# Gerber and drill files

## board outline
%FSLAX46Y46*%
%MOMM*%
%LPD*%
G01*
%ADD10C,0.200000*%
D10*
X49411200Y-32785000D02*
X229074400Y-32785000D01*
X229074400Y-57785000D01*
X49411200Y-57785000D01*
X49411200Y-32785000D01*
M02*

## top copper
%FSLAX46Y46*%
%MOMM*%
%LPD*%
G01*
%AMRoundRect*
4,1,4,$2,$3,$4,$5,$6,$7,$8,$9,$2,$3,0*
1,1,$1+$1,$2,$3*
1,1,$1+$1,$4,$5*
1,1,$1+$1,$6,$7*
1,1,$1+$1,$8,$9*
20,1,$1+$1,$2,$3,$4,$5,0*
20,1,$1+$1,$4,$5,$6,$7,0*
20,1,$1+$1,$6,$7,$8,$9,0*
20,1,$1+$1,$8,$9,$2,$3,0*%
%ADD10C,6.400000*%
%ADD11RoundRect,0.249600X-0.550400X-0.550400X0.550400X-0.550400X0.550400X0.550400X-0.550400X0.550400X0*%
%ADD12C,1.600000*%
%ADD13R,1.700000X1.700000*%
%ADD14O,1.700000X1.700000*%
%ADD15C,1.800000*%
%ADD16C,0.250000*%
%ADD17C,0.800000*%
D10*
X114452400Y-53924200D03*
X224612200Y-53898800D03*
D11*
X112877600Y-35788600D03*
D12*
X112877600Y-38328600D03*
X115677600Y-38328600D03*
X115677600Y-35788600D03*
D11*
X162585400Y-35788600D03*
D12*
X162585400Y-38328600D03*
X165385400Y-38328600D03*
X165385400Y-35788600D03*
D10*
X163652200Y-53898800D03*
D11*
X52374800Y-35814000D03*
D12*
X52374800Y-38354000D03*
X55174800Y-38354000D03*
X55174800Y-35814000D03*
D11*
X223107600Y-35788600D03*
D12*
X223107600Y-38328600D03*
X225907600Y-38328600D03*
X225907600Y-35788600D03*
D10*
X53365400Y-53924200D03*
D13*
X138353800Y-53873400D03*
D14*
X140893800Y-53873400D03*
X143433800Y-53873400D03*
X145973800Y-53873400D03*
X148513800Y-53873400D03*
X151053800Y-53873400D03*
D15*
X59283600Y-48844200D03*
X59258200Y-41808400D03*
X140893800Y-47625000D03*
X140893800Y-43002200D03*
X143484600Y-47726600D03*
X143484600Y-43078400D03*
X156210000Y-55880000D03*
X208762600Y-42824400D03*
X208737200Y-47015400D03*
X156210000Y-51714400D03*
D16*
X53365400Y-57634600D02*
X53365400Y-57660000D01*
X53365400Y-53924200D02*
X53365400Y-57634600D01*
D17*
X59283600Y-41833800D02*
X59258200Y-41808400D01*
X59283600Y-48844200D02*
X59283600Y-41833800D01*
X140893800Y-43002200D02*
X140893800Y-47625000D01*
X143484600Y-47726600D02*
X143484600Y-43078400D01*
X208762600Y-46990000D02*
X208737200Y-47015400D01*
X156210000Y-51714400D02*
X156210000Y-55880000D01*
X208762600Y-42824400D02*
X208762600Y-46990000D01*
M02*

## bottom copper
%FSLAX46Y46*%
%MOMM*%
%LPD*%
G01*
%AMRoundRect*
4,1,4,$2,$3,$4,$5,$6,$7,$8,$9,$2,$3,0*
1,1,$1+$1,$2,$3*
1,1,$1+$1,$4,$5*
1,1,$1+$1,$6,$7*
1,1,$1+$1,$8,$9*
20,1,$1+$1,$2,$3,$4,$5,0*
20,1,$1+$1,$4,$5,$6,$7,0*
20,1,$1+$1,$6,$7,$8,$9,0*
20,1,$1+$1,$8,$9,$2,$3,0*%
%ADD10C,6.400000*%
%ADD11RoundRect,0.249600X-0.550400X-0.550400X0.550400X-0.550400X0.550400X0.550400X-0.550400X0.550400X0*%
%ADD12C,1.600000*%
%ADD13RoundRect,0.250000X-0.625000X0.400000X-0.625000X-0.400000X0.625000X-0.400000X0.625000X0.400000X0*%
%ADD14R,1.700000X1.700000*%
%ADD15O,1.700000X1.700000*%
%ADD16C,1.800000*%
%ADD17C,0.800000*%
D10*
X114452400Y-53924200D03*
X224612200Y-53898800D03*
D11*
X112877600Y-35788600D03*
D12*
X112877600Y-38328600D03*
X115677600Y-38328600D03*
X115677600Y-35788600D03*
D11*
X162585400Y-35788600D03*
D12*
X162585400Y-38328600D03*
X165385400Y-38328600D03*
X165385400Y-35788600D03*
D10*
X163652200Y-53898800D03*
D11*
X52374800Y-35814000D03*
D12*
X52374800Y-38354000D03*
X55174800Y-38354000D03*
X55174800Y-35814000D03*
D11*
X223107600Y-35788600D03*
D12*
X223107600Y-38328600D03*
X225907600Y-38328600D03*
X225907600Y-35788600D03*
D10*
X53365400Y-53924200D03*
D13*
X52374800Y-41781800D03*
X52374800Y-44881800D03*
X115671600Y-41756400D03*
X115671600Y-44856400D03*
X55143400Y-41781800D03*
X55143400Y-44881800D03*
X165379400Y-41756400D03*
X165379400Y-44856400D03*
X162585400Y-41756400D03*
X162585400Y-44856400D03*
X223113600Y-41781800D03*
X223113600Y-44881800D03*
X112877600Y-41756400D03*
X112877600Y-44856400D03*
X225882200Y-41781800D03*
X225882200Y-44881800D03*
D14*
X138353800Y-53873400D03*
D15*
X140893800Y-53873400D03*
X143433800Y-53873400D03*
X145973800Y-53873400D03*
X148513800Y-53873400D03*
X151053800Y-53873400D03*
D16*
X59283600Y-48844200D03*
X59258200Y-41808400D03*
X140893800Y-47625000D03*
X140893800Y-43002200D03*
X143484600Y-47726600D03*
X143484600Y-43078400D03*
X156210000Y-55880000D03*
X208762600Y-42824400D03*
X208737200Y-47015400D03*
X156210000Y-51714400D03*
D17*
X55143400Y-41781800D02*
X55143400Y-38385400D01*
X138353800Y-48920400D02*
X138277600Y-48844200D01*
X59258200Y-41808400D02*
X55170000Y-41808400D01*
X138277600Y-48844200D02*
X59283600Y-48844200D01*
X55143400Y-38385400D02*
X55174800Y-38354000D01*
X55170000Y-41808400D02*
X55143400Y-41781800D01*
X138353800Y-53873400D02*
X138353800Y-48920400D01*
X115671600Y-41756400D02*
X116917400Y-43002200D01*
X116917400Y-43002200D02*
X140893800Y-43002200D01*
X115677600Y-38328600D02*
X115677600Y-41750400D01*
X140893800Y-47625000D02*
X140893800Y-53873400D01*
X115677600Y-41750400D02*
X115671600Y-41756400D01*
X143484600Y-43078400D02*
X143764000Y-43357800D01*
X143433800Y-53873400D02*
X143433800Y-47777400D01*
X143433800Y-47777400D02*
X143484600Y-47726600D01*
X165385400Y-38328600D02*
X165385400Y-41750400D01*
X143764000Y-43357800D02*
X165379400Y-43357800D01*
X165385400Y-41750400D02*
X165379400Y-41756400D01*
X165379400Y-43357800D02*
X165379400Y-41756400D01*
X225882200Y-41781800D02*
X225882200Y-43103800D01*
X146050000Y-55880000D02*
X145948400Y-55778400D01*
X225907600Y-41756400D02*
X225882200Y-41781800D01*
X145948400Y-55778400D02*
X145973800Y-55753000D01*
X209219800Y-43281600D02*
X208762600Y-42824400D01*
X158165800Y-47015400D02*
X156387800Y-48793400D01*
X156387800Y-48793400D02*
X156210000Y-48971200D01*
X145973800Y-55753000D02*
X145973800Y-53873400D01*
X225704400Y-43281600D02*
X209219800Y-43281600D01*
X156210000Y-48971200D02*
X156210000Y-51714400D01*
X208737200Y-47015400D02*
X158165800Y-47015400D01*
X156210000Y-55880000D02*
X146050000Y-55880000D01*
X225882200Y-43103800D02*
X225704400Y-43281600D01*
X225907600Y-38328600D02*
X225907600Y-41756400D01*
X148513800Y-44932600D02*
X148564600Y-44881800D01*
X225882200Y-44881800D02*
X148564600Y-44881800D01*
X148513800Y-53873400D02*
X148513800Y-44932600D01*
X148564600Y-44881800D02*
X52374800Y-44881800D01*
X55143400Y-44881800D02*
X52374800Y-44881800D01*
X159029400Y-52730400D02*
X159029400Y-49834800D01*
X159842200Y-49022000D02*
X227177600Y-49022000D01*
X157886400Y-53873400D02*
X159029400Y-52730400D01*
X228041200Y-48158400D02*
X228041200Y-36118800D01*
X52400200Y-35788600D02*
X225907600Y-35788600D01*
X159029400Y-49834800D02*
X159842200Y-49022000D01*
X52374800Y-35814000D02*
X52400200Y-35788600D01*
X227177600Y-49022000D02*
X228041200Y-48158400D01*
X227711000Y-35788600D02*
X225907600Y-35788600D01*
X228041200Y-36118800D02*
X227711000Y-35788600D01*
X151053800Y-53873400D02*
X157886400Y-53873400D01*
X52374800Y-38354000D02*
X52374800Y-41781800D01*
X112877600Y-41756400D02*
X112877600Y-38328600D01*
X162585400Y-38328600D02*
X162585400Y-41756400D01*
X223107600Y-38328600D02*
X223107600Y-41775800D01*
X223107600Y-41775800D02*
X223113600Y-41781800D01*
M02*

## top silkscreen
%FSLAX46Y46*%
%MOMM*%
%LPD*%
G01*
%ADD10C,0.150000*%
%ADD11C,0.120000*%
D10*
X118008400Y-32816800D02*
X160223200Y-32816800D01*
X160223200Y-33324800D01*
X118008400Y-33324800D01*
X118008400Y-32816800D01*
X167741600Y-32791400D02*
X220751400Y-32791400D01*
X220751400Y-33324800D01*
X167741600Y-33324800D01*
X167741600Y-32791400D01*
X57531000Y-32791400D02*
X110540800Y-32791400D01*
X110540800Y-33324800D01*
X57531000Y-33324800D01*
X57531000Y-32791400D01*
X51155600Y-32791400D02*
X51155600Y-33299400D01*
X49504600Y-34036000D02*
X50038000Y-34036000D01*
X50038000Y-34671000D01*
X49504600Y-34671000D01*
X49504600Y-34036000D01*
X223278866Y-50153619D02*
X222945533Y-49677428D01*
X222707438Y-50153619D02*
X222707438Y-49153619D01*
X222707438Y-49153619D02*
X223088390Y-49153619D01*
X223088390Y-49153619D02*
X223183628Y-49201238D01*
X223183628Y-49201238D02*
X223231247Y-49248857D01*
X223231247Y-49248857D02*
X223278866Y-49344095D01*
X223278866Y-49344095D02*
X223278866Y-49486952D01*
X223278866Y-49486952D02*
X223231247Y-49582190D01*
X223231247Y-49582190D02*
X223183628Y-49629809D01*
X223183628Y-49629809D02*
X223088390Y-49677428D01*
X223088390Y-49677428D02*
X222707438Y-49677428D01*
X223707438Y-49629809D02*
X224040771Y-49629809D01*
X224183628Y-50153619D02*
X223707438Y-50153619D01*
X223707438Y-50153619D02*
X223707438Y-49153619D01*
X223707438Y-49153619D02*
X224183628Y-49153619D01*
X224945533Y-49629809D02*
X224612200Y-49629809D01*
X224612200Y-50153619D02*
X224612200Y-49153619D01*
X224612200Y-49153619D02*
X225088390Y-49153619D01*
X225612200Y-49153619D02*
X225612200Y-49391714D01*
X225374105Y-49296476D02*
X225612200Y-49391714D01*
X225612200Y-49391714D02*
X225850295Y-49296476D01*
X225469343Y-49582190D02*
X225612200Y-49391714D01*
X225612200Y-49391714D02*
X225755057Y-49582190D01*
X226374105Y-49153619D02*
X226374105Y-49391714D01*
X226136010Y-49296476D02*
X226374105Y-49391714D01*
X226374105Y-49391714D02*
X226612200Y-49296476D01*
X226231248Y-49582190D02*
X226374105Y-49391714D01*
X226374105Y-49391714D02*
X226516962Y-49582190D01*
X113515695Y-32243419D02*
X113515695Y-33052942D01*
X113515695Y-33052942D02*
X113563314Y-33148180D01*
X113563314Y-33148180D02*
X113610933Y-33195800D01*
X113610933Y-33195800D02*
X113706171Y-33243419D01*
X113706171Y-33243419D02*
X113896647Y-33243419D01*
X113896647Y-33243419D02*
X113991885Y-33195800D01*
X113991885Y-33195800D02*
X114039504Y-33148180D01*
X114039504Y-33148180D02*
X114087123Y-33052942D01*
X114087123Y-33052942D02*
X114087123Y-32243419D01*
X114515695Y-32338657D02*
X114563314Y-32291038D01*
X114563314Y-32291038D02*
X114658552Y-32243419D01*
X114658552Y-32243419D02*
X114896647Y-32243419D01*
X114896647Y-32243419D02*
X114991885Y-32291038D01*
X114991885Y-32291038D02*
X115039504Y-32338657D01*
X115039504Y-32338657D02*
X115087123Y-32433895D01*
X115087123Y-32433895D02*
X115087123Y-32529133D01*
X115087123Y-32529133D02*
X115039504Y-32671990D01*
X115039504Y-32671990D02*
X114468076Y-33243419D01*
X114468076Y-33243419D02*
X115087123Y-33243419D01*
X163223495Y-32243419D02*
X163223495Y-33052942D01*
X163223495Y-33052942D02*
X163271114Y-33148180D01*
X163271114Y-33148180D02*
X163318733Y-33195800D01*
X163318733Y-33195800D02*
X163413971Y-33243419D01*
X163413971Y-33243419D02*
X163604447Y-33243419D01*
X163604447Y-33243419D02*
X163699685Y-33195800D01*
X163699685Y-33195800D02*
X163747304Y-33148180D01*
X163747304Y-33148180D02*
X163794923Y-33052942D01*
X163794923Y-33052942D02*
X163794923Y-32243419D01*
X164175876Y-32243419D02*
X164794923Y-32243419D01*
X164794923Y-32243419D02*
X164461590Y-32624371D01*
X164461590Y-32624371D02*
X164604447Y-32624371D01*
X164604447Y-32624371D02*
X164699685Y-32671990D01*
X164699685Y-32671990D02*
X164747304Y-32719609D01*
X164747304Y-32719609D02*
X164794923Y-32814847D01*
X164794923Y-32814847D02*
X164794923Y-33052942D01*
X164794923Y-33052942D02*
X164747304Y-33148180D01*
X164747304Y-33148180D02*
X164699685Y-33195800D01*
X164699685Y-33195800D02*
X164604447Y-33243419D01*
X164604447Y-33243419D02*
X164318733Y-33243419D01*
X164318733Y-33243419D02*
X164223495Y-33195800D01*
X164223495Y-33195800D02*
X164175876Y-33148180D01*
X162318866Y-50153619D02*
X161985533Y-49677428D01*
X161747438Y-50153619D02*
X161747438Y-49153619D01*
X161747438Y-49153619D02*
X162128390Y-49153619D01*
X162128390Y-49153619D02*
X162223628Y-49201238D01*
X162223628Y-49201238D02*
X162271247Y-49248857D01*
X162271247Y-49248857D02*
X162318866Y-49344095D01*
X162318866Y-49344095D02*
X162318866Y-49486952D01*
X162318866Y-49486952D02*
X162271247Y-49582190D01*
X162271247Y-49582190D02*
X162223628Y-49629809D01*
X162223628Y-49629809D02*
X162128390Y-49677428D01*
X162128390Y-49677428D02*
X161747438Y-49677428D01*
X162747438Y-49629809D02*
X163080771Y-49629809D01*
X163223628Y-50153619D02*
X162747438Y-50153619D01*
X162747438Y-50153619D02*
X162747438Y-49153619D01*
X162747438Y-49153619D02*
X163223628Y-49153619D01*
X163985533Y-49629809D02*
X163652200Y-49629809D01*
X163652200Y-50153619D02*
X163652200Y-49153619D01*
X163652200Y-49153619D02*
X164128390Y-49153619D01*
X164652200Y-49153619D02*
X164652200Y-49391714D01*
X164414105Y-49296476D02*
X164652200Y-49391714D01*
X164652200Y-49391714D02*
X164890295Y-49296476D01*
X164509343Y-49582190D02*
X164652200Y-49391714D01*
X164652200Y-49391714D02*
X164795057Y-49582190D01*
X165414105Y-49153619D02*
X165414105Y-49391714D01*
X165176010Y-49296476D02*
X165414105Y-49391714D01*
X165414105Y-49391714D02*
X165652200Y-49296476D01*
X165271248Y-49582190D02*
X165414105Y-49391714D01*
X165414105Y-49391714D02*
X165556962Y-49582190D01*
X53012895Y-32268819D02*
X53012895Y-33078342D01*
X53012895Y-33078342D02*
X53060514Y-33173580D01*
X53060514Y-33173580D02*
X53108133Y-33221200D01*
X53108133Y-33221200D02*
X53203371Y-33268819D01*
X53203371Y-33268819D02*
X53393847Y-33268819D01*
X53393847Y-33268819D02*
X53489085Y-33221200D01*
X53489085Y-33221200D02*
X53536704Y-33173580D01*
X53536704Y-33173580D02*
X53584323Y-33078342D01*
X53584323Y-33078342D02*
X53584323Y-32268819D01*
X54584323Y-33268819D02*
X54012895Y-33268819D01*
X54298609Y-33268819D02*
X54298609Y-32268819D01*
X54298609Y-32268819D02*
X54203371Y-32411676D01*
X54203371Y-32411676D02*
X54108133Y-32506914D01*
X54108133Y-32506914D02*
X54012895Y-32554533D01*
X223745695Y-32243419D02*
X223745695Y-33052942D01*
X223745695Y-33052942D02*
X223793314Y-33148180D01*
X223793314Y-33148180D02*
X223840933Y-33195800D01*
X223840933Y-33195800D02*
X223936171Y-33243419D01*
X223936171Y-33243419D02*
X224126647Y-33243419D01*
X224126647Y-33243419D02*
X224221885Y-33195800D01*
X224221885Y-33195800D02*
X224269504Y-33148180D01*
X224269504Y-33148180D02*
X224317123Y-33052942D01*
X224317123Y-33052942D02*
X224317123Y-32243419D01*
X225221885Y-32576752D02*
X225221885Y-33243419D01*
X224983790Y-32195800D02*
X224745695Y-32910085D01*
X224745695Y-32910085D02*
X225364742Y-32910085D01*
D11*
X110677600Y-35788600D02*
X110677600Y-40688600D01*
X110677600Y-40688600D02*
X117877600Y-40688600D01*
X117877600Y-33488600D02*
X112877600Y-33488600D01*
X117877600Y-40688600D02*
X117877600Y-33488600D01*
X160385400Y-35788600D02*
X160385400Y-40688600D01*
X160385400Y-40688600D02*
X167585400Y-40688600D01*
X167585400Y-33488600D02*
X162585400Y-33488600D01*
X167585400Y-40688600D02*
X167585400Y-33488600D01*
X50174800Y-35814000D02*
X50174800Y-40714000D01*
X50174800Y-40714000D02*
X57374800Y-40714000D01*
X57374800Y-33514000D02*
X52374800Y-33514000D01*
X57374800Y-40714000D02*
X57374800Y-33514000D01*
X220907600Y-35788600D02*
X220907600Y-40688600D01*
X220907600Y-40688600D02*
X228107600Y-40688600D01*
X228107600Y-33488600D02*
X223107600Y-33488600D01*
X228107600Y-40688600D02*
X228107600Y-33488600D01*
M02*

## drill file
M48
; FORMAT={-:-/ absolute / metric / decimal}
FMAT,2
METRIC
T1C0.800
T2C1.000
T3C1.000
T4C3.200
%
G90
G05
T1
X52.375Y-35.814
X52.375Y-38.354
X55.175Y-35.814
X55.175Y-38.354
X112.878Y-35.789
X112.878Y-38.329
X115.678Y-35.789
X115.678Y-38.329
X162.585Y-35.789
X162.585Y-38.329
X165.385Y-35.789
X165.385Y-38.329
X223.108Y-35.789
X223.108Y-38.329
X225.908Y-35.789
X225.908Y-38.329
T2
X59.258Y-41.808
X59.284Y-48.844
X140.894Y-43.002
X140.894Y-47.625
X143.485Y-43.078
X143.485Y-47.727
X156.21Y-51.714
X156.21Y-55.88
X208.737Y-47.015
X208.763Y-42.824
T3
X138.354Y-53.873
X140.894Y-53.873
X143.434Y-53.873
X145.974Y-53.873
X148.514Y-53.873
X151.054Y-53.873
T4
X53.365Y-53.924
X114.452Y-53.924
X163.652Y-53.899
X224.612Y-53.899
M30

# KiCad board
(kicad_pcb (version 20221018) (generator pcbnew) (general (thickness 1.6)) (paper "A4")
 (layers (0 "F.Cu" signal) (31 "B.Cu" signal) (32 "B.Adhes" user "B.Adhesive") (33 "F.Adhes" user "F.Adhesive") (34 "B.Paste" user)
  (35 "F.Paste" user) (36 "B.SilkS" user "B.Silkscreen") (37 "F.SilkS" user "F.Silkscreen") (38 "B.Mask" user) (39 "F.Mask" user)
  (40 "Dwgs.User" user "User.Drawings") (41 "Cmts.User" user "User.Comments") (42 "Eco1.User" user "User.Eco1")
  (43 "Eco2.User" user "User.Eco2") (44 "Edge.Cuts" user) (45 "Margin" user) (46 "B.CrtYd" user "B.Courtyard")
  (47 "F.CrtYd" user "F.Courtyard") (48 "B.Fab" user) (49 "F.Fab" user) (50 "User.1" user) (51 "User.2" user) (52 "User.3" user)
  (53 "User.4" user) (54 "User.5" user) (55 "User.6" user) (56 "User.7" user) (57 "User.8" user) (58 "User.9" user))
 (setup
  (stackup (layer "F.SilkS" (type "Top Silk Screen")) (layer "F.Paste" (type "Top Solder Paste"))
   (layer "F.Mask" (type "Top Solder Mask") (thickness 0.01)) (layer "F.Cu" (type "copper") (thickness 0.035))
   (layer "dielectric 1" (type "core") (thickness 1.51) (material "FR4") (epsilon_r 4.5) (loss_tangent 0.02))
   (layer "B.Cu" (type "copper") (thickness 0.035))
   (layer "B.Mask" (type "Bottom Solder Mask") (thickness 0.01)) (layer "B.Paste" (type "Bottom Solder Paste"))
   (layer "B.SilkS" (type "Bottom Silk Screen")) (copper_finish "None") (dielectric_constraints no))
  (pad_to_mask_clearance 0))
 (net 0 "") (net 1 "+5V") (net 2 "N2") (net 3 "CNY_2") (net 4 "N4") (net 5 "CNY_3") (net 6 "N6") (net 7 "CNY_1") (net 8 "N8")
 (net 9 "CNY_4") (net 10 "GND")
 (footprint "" (layer "F.Cu") (at 114.4524 53.9242)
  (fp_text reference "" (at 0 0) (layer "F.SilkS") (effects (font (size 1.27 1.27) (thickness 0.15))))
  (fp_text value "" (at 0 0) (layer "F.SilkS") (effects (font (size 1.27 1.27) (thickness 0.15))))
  (pad "1" thru_hole circle (at 0 0) (size 6.4 6.4) (drill 3.2) (layers "*.Cu" "*.Mask")))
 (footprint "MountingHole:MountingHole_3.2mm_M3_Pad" (layer "F.Cu") (at 224.6122 53.8988)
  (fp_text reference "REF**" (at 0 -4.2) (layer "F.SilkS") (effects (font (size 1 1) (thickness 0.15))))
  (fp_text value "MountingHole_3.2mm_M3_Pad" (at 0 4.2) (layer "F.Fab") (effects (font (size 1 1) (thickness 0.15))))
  (pad "1" thru_hole circle (at 0 0) (size 6.4 6.4) (drill 3.2) (layers "*.Cu" "*.Mask")))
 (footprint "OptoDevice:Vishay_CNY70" (layer "F.Cu") (at 112.8776 35.7886)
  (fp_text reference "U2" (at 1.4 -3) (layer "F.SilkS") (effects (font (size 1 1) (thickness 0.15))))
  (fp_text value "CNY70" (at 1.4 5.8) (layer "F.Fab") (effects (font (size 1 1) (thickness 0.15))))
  (fp_line (start -2.2 0) (end -2.2 4.9) (stroke (width 0.12) (type solid)) (layer "F.SilkS"))
  (fp_line (start -2.2 4.9) (end 5 4.9) (stroke (width 0.12) (type solid)) (layer "F.SilkS"))
  (fp_line (start 5 -2.3) (end 0 -2.3) (stroke (width 0.12) (type solid)) (layer "F.SilkS"))
  (fp_line (start 5 4.9) (end 5 -2.3) (stroke (width 0.12) (type solid)) (layer "F.SilkS"))
  (pad "1" thru_hole roundrect (at 0 0) (size 1.6 1.6) (drill 0.8) (layers "*.Cu" "*.Mask") (roundrect_rratio 0.156) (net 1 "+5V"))
  (pad "2" thru_hole circle (at 0 2.54) (size 1.6 1.6) (drill 0.8) (layers "*.Cu" "*.Mask") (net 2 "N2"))
  (pad "3" thru_hole circle (at 2.8 2.54) (size 1.6 1.6) (drill 0.8) (layers "*.Cu" "*.Mask") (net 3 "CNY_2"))
  (pad "4" thru_hole circle (at 2.8 0) (size 1.6 1.6) (drill 0.8) (layers "*.Cu" "*.Mask") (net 1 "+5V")))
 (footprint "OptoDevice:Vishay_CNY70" (layer "F.Cu") (at 162.5854 35.7886)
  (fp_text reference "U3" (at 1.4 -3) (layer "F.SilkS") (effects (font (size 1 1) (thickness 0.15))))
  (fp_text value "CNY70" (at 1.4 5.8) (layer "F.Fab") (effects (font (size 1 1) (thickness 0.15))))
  (fp_line (start -2.2 0) (end -2.2 4.9) (stroke (width 0.12) (type solid)) (layer "F.SilkS"))
  (fp_line (start -2.2 4.9) (end 5 4.9) (stroke (width 0.12) (type solid)) (layer "F.SilkS"))
  (fp_line (start 5 -2.3) (end 0 -2.3) (stroke (width 0.12) (type solid)) (layer "F.SilkS"))
  (fp_line (start 5 4.9) (end 5 -2.3) (stroke (width 0.12) (type solid)) (layer "F.SilkS"))
  (pad "1" thru_hole roundrect (at 0 0) (size 1.6 1.6) (drill 0.8) (layers "*.Cu" "*.Mask") (roundrect_rratio 0.156) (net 1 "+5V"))
  (pad "2" thru_hole circle (at 0 2.54) (size 1.6 1.6) (drill 0.8) (layers "*.Cu" "*.Mask") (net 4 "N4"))
  (pad "3" thru_hole circle (at 2.8 2.54) (size 1.6 1.6) (drill 0.8) (layers "*.Cu" "*.Mask") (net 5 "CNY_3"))
  (pad "4" thru_hole circle (at 2.8 0) (size 1.6 1.6) (drill 0.8) (layers "*.Cu" "*.Mask") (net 1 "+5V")))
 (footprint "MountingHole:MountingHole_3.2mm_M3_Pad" (layer "F.Cu") (at 163.6522 53.8988)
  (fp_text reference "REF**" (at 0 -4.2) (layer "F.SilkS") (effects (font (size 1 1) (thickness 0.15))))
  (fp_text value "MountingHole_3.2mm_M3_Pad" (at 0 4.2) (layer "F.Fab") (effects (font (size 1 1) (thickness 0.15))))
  (pad "1" thru_hole circle (at 0 0) (size 6.4 6.4) (drill 3.2) (layers "*.Cu" "*.Mask")))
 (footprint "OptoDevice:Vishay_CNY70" (layer "F.Cu") (at 52.3748 35.814)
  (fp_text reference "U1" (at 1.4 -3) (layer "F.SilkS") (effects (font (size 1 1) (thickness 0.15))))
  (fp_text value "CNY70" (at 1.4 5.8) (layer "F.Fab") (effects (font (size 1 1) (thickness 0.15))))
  (fp_line (start -2.2 0) (end -2.2 4.9) (stroke (width 0.12) (type solid)) (layer "F.SilkS"))
  (fp_line (start -2.2 4.9) (end 5 4.9) (stroke (width 0.12) (type solid)) (layer "F.SilkS"))
  (fp_line (start 5 -2.3) (end 0 -2.3) (stroke (width 0.12) (type solid)) (layer "F.SilkS"))
  (fp_line (start 5 4.9) (end 5 -2.3) (stroke (width 0.12) (type solid)) (layer "F.SilkS"))
  (pad "1" thru_hole roundrect (at 0 0) (size 1.6 1.6) (drill 0.8) (layers "*.Cu" "*.Mask") (roundrect_rratio 0.156) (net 1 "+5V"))
  (pad "2" thru_hole circle (at 0 2.54) (size 1.6 1.6) (drill 0.8) (layers "*.Cu" "*.Mask") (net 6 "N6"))
  (pad "3" thru_hole circle (at 2.8 2.54) (size 1.6 1.6) (drill 0.8) (layers "*.Cu" "*.Mask") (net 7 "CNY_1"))
  (pad "4" thru_hole circle (at 2.8 0) (size 1.6 1.6) (drill 0.8) (layers "*.Cu" "*.Mask") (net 1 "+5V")))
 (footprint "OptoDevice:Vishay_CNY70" (layer "F.Cu") (at 223.1076 35.7886)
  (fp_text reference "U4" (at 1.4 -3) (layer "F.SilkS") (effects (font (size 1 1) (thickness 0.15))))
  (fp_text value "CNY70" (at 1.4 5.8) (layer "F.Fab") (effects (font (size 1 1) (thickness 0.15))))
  (fp_line (start -2.2 0) (end -2.2 4.9) (stroke (width 0.12) (type solid)) (layer "F.SilkS"))
  (fp_line (start -2.2 4.9) (end 5 4.9) (stroke (width 0.12) (type solid)) (layer "F.SilkS"))
  (fp_line (start 5 -2.3) (end 0 -2.3) (stroke (width 0.12) (type solid)) (layer "F.SilkS"))
  (fp_line (start 5 4.9) (end 5 -2.3) (stroke (width 0.12) (type solid)) (layer "F.SilkS"))
  (pad "1" thru_hole roundrect (at 0 0) (size 1.6 1.6) (drill 0.8) (layers "*.Cu" "*.Mask") (roundrect_rratio 0.156) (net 1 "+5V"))
  (pad "2" thru_hole circle (at 0 2.54) (size 1.6 1.6) (drill 0.8) (layers "*.Cu" "*.Mask") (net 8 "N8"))
  (pad "3" thru_hole circle (at 2.8 2.54) (size 1.6 1.6) (drill 0.8) (layers "*.Cu" "*.Mask") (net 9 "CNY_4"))
  (pad "4" thru_hole circle (at 2.8 0) (size 1.6 1.6) (drill 0.8) (layers "*.Cu" "*.Mask") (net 1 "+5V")))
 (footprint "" (layer "F.Cu") (at 53.3654 53.9242)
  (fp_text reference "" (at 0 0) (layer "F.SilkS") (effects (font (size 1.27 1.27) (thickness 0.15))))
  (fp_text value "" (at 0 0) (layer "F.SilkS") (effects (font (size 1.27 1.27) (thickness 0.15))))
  (pad "1" thru_hole circle (at 0 0) (size 6.4 6.4) (drill 3.2) (layers "*.Cu" "*.Mask")))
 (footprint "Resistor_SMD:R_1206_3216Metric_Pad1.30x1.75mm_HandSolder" (layer "B.Cu") (at 52.3748 43.3318 -90)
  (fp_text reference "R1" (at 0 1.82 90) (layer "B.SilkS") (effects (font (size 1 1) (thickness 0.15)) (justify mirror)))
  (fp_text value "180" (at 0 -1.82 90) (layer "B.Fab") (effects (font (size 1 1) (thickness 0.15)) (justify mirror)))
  (pad "1" smd roundrect (at -1.55 0 270) (size 1.3 1.75) (layers "B.Cu" "B.Paste" "B.Mask") (roundrect_rratio 0.192308) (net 6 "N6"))
  (pad "2" smd roundrect (at 1.55 0 270) (size 1.3 1.75) (layers "B.Cu" "B.Paste" "B.Mask") (roundrect_rratio 0.192308) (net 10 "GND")))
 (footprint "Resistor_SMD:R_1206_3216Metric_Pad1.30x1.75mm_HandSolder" (layer "B.Cu") (at 115.6716 43.3064 -90)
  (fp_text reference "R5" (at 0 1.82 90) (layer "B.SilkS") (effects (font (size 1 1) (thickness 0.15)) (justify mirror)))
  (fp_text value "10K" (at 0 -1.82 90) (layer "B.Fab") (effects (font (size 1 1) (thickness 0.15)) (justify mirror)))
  (pad "1" smd roundrect (at -1.55 0 270) (size 1.3 1.75) (layers "B.Cu" "B.Paste" "B.Mask") (roundrect_rratio 0.192308) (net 3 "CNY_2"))
  (pad "2" smd roundrect (at 1.55 0 270) (size 1.3 1.75) (layers "B.Cu" "B.Paste" "B.Mask") (roundrect_rratio 0.192308) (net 10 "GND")))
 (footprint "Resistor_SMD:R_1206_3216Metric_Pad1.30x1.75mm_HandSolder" (layer "B.Cu") (at 55.1434 43.3318 -90)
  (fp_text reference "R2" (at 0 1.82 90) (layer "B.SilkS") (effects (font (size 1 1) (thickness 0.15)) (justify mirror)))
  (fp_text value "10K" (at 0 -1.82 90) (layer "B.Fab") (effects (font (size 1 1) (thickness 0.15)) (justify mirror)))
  (pad "1" smd roundrect (at -1.55 0 270) (size 1.3 1.75) (layers "B.Cu" "B.Paste" "B.Mask") (roundrect_rratio 0.192308) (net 7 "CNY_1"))
  (pad "2" smd roundrect (at 1.55 0 270) (size 1.3 1.75) (layers "B.Cu" "B.Paste" "B.Mask") (roundrect_rratio 0.192308) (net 10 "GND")))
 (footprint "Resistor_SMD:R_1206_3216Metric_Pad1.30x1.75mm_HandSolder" (layer "B.Cu") (at 165.3794 43.3064 -90)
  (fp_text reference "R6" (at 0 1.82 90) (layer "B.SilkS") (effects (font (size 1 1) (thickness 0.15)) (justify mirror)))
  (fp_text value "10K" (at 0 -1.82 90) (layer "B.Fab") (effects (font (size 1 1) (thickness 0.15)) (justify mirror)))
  (pad "1" smd roundrect (at -1.55 0 270) (size 1.3 1.75) (layers "B.Cu" "B.Paste" "B.Mask") (roundrect_rratio 0.192308) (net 5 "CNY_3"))
  (pad "2" smd roundrect (at 1.55 0 270) (size 1.3 1.75) (layers "B.Cu" "B.Paste" "B.Mask") (roundrect_rratio 0.192308) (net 10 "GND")))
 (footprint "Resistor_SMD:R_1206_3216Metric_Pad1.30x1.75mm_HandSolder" (layer "B.Cu") (at 162.5854 43.3064 -90)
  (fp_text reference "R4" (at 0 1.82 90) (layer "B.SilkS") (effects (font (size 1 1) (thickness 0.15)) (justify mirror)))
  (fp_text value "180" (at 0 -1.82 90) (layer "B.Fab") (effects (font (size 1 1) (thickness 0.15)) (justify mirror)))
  (pad "1" smd roundrect (at -1.55 0 270) (size 1.3 1.75) (layers "B.Cu" "B.Paste" "B.Mask") (roundrect_rratio 0.192308) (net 4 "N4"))
  (pad "2" smd roundrect (at 1.55 0 270) (size 1.3 1.75) (layers "B.Cu" "B.Paste" "B.Mask") (roundrect_rratio 0.192308) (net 10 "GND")))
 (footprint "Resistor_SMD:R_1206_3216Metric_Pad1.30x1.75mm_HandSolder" (layer "B.Cu") (at 223.1136 43.3318 -90)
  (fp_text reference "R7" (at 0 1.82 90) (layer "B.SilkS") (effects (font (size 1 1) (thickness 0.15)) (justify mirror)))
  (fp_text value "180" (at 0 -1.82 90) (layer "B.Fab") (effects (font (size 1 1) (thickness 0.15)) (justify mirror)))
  (pad "1" smd roundrect (at -1.55 0 270) (size 1.3 1.75) (layers "B.Cu" "B.Paste" "B.Mask") (roundrect_rratio 0.192308) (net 8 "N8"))
  (pad "2" smd roundrect (at 1.55 0 270) (size 1.3 1.75) (layers "B.Cu" "B.Paste" "B.Mask") (roundrect_rratio 0.192308) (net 10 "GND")))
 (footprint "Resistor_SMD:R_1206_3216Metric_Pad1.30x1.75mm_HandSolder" (layer "B.Cu") (at 112.8776 43.3064 -90)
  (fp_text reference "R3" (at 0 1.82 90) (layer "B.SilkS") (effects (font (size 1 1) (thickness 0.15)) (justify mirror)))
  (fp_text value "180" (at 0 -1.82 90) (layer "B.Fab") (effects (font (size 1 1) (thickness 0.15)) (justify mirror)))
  (pad "1" smd roundrect (at -1.55 0 270) (size 1.3 1.75) (layers "B.Cu" "B.Paste" "B.Mask") (roundrect_rratio 0.192308) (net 2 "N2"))
  (pad "2" smd roundrect (at 1.55 0 270) (size 1.3 1.75) (layers "B.Cu" "B.Paste" "B.Mask") (roundrect_rratio 0.192308) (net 10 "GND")))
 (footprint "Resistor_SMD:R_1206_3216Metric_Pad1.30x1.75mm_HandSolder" (layer "B.Cu") (at 225.8822 43.3318 -90)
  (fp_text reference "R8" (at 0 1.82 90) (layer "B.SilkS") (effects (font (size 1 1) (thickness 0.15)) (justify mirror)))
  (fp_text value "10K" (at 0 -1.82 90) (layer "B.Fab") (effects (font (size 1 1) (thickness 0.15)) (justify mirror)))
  (pad "1" smd roundrect (at -1.55 0 270) (size 1.3 1.75) (layers "B.Cu" "B.Paste" "B.Mask") (roundrect_rratio 0.192308) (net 9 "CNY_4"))
  (pad "2" smd roundrect (at 1.55 0 270) (size 1.3 1.75) (layers "B.Cu" "B.Paste" "B.Mask") (roundrect_rratio 0.192308) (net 10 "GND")))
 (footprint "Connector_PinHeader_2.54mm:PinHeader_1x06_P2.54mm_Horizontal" (layer "B.Cu") (at 138.3538 53.8734 -90)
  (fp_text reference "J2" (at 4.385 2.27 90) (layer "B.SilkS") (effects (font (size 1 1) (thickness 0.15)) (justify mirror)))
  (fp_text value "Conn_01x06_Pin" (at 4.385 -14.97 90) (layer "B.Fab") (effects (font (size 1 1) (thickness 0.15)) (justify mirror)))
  (pad "1" thru_hole rect (at 0 0 270) (size 1.7 1.7) (drill 1) (layers "*.Cu" "*.Mask") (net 7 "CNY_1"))
  (pad "2" thru_hole oval (at 0 -2.54 270) (size 1.7 1.7) (drill 1) (layers "*.Cu" "*.Mask") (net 3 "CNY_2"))
  (pad "3" thru_hole oval (at 0 -5.08 270) (size 1.7 1.7) (drill 1) (layers "*.Cu" "*.Mask") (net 5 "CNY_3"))
  (pad "4" thru_hole oval (at 0 -7.62 270) (size 1.7 1.7) (drill 1) (layers "*.Cu" "*.Mask") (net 9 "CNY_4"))
  (pad "5" thru_hole oval (at 0 -10.16 270) (size 1.7 1.7) (drill 1) (layers "*.Cu" "*.Mask") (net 10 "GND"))
  (pad "6" thru_hole oval (at 0 -12.7 270) (size 1.7 1.7) (drill 1) (layers "*.Cu" "*.Mask") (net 1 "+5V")))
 (gr_rect (start 118.0084 32.8168) (end 160.2232 33.3248) (stroke (width 0.15) (type default)) (fill none) (layer "F.SilkS"))
 (gr_rect (start 167.7416 32.7914) (end 220.7514 33.3248) (stroke (width 0.15) (type default)) (fill none) (layer "F.SilkS"))
 (gr_rect (start 57.531 32.7914) (end 110.5408 33.3248) (stroke (width 0.15) (type default)) (fill none) (layer "F.SilkS"))
 (gr_line (start 51.1556 32.7914) (end 51.1556 33.2994) (stroke (width 0.15) (type default)) (layer "F.SilkS"))
 (gr_rect (start 49.5046 34.036) (end 50.038 34.671) (stroke (width 0.15) (type default)) (fill none) (layer "F.SilkS"))
 (gr_rect (start 49.4112 32.785) (end 229.0744 57.785) (stroke (width 0.2) (type default)) (fill none) (layer "Edge.Cuts"))
 (segment (start 53.3654 57.6346) (end 53.3654 57.66) (width 0.25) (layer "F.Cu") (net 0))
 (segment (start 53.3654 53.9242) (end 53.3654 57.6346) (width 0.25) (layer "F.Cu") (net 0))
 (segment (start 59.2836 41.8338) (end 59.2582 41.8084) (width 0.8) (layer "F.Cu") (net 7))
 (segment (start 59.2836 48.8442) (end 59.2836 41.8338) (width 0.8) (layer "F.Cu") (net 7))
 (via (at 59.2836 48.8442) (size 1.8) (drill 1) (layers "F.Cu" "B.Cu") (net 7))
 (via (at 59.2582 41.8084) (size 1.8) (drill 1) (layers "F.Cu" "B.Cu") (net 7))
 (segment (start 55.1434 41.7818) (end 55.1434 38.3854) (width 0.8) (layer "B.Cu") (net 7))
 (segment (start 138.3538 48.9204) (end 138.2776 48.8442) (width 0.8) (layer "B.Cu") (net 7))
 (segment (start 59.2582 41.8084) (end 55.17 41.8084) (width 0.8) (layer "B.Cu") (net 7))
 (segment (start 138.2776 48.8442) (end 59.2836 48.8442) (width 0.8) (layer "B.Cu") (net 7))
 (segment (start 55.1434 38.3854) (end 55.1748 38.354) (width 0.8) (layer "B.Cu") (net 7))
 (segment (start 55.17 41.8084) (end 55.1434 41.7818) (width 0.8) (layer "B.Cu") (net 7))
 (segment (start 138.3538 53.8734) (end 138.3538 48.9204) (width 0.8) (layer "B.Cu") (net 7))
 (segment (start 140.8938 43.0022) (end 140.8938 47.625) (width 0.8) (layer "F.Cu") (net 3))
 (via (at 140.8938 47.625) (size 1.8) (drill 1) (layers "F.Cu" "B.Cu") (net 3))
 (via (at 140.8938 43.0022) (size 1.8) (drill 1) (layers "F.Cu" "B.Cu") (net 3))
 (segment (start 115.6716 41.7564) (end 116.9174 43.0022) (width 0.8) (layer "B.Cu") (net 3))
 (segment (start 116.9174 43.0022) (end 140.8938 43.0022) (width 0.8) (layer "B.Cu") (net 3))
 (segment (start 115.6776 38.3286) (end 115.6776 41.7504) (width 0.8) (layer "B.Cu") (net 3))
 (segment (start 140.8938 47.625) (end 140.8938 53.8734) (width 0.8) (layer "B.Cu") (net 3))
 (segment (start 115.6776 41.7504) (end 115.6716 41.7564) (width 0.8) (layer "B.Cu") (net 3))
 (segment (start 143.4846 47.7266) (end 143.4846 43.0784) (width 0.8) (layer "F.Cu") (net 5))
 (via (at 143.4846 47.7266) (size 1.8) (drill 1) (layers "F.Cu" "B.Cu") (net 5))
 (via (at 143.4846 43.0784) (size 1.8) (drill 1) (layers "F.Cu" "B.Cu") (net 5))
 (segment (start 143.4846 43.0784) (end 143.764 43.3578) (width 0.8) (layer "B.Cu") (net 5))
 (segment (start 143.4338 53.8734) (end 143.4338 47.7774) (width 0.8) (layer "B.Cu") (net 5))
 (segment (start 143.4338 47.7774) (end 143.4846 47.7266) (width 0.8) (layer "B.Cu") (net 5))
 (segment (start 165.3854 38.3286) (end 165.3854 41.7504) (width 0.8) (layer "B.Cu") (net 5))
 (segment (start 143.764 43.3578) (end 165.3794 43.3578) (width 0.8) (layer "B.Cu") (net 5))
 (segment (start 165.3854 41.7504) (end 165.3794 41.7564) (width 0.8) (layer "B.Cu") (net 5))
 (segment (start 165.3794 43.3578) (end 165.3794 41.7564) (width 0.8) (layer "B.Cu") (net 5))
 (segment (start 208.7626 46.99) (end 208.7372 47.0154) (width 0.8) (layer "F.Cu") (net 9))
 (segment (start 156.21 51.7144) (end 156.21 55.88) (width 0.8) (layer "F.Cu") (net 9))
 (segment (start 208.7626 42.8244) (end 208.7626 46.99) (width 0.8) (layer "F.Cu") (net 9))
 (via (at 156.21 55.88) (size 1.8) (drill 1) (layers "F.Cu" "B.Cu") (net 9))
 (via (at 208.7626 42.8244) (size 1.8) (drill 1) (layers "F.Cu" "B.Cu") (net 9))
 (via (at 208.7372 47.0154) (size 1.8) (drill 1) (layers "F.Cu" "B.Cu") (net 9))
 (via (at 156.21 51.7144) (size 1.8) (drill 1) (layers "F.Cu" "B.Cu") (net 9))
 (segment (start 225.8822 41.7818) (end 225.8822 43.1038) (width 0.8) (layer "B.Cu") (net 9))
 (segment (start 146.05 55.88) (end 145.9484 55.7784) (width 0.8) (layer "B.Cu") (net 9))
 (segment (start 225.9076 41.7564) (end 225.8822 41.7818) (width 0.8) (layer "B.Cu") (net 9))
 (segment (start 145.9484 55.7784) (end 145.9738 55.753) (width 0.8) (layer "B.Cu") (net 9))
 (segment (start 209.2198 43.2816) (end 208.7626 42.8244) (width 0.8) (layer "B.Cu") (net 9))
 (segment (start 158.1658 47.0154) (end 156.3878 48.7934) (width 0.8) (layer "B.Cu") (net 9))
 (segment (start 156.3878 48.7934) (end 156.21 48.9712) (width 0.8) (layer "B.Cu") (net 9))
 (segment (start 145.9738 55.753) (end 145.9738 53.8734) (width 0.8) (layer "B.Cu") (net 9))
 (segment (start 225.7044 43.2816) (end 209.2198 43.2816) (width 0.8) (layer "B.Cu") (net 9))
 (segment (start 156.21 48.9712) (end 156.21 51.7144) (width 0.8) (layer "B.Cu") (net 9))
 (segment (start 208.7372 47.0154) (end 158.1658 47.0154) (width 0.8) (layer "B.Cu") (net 9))
 (segment (start 156.21 55.88) (end 146.05 55.88) (width 0.8) (layer "B.Cu") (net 9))
 (segment (start 225.8822 43.1038) (end 225.7044 43.2816) (width 0.8) (layer "B.Cu") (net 9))
 (segment (start 225.9076 38.3286) (end 225.9076 41.7564) (width 0.8) (layer "B.Cu") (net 9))
 (segment (start 148.5138 44.9326) (end 148.5646 44.8818) (width 0.8) (layer "B.Cu") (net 10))
 (segment (start 225.8822 44.8818) (end 148.5646 44.8818) (width 0.8) (layer "B.Cu") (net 10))
 (segment (start 148.5138 53.8734) (end 148.5138 44.9326) (width 0.8) (layer "B.Cu") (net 10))
 (segment (start 148.5646 44.8818) (end 52.3748 44.8818) (width 0.8) (layer "B.Cu") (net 10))
 (segment (start 55.1434 44.8818) (end 52.3748 44.8818) (width 0.8) (layer "B.Cu") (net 10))
 (segment (start 159.0294 52.7304) (end 159.0294 49.8348) (width 0.8) (layer "B.Cu") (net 1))
 (segment (start 159.8422 49.022) (end 227.1776 49.022) (width 0.8) (layer "B.Cu") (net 1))
 (segment (start 157.8864 53.8734) (end 159.0294 52.7304) (width 0.8) (layer "B.Cu") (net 1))
 (segment (start 228.0412 48.1584) (end 228.0412 36.1188) (width 0.8) (layer "B.Cu") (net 1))
 (segment (start 52.4002 35.7886) (end 225.9076 35.7886) (width 0.8) (layer "B.Cu") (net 1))
 (segment (start 159.0294 49.8348) (end 159.8422 49.022) (width 0.8) (layer "B.Cu") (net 1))
 (segment (start 52.3748 35.814) (end 52.4002 35.7886) (width 0.8) (layer "B.Cu") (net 1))
 (segment (start 227.1776 49.022) (end 228.0412 48.1584) (width 0.8) (layer "B.Cu") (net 1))
 (segment (start 227.711 35.7886) (end 225.9076 35.7886) (width 0.8) (layer "B.Cu") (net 1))
 (segment (start 228.0412 36.1188) (end 227.711 35.7886) (width 0.8) (layer "B.Cu") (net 1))
 (segment (start 151.0538 53.8734) (end 157.8864 53.8734) (width 0.8) (layer "B.Cu") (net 1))
 (segment (start 52.3748 38.354) (end 52.3748 41.7818) (width 0.8) (layer "B.Cu") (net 6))
 (segment (start 112.8776 41.7564) (end 112.8776 38.3286) (width 0.8) (layer "B.Cu") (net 2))
 (segment (start 162.5854 38.3286) (end 162.5854 41.7564) (width 0.8) (layer "B.Cu") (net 4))
 (segment (start 223.1076 38.3286) (end 223.1076 41.7758) (width 0.8) (layer "B.Cu") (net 8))
 (segment (start 223.1076 41.7758) (end 223.1136 41.7818) (width 0.8) (layer "B.Cu") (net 8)))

